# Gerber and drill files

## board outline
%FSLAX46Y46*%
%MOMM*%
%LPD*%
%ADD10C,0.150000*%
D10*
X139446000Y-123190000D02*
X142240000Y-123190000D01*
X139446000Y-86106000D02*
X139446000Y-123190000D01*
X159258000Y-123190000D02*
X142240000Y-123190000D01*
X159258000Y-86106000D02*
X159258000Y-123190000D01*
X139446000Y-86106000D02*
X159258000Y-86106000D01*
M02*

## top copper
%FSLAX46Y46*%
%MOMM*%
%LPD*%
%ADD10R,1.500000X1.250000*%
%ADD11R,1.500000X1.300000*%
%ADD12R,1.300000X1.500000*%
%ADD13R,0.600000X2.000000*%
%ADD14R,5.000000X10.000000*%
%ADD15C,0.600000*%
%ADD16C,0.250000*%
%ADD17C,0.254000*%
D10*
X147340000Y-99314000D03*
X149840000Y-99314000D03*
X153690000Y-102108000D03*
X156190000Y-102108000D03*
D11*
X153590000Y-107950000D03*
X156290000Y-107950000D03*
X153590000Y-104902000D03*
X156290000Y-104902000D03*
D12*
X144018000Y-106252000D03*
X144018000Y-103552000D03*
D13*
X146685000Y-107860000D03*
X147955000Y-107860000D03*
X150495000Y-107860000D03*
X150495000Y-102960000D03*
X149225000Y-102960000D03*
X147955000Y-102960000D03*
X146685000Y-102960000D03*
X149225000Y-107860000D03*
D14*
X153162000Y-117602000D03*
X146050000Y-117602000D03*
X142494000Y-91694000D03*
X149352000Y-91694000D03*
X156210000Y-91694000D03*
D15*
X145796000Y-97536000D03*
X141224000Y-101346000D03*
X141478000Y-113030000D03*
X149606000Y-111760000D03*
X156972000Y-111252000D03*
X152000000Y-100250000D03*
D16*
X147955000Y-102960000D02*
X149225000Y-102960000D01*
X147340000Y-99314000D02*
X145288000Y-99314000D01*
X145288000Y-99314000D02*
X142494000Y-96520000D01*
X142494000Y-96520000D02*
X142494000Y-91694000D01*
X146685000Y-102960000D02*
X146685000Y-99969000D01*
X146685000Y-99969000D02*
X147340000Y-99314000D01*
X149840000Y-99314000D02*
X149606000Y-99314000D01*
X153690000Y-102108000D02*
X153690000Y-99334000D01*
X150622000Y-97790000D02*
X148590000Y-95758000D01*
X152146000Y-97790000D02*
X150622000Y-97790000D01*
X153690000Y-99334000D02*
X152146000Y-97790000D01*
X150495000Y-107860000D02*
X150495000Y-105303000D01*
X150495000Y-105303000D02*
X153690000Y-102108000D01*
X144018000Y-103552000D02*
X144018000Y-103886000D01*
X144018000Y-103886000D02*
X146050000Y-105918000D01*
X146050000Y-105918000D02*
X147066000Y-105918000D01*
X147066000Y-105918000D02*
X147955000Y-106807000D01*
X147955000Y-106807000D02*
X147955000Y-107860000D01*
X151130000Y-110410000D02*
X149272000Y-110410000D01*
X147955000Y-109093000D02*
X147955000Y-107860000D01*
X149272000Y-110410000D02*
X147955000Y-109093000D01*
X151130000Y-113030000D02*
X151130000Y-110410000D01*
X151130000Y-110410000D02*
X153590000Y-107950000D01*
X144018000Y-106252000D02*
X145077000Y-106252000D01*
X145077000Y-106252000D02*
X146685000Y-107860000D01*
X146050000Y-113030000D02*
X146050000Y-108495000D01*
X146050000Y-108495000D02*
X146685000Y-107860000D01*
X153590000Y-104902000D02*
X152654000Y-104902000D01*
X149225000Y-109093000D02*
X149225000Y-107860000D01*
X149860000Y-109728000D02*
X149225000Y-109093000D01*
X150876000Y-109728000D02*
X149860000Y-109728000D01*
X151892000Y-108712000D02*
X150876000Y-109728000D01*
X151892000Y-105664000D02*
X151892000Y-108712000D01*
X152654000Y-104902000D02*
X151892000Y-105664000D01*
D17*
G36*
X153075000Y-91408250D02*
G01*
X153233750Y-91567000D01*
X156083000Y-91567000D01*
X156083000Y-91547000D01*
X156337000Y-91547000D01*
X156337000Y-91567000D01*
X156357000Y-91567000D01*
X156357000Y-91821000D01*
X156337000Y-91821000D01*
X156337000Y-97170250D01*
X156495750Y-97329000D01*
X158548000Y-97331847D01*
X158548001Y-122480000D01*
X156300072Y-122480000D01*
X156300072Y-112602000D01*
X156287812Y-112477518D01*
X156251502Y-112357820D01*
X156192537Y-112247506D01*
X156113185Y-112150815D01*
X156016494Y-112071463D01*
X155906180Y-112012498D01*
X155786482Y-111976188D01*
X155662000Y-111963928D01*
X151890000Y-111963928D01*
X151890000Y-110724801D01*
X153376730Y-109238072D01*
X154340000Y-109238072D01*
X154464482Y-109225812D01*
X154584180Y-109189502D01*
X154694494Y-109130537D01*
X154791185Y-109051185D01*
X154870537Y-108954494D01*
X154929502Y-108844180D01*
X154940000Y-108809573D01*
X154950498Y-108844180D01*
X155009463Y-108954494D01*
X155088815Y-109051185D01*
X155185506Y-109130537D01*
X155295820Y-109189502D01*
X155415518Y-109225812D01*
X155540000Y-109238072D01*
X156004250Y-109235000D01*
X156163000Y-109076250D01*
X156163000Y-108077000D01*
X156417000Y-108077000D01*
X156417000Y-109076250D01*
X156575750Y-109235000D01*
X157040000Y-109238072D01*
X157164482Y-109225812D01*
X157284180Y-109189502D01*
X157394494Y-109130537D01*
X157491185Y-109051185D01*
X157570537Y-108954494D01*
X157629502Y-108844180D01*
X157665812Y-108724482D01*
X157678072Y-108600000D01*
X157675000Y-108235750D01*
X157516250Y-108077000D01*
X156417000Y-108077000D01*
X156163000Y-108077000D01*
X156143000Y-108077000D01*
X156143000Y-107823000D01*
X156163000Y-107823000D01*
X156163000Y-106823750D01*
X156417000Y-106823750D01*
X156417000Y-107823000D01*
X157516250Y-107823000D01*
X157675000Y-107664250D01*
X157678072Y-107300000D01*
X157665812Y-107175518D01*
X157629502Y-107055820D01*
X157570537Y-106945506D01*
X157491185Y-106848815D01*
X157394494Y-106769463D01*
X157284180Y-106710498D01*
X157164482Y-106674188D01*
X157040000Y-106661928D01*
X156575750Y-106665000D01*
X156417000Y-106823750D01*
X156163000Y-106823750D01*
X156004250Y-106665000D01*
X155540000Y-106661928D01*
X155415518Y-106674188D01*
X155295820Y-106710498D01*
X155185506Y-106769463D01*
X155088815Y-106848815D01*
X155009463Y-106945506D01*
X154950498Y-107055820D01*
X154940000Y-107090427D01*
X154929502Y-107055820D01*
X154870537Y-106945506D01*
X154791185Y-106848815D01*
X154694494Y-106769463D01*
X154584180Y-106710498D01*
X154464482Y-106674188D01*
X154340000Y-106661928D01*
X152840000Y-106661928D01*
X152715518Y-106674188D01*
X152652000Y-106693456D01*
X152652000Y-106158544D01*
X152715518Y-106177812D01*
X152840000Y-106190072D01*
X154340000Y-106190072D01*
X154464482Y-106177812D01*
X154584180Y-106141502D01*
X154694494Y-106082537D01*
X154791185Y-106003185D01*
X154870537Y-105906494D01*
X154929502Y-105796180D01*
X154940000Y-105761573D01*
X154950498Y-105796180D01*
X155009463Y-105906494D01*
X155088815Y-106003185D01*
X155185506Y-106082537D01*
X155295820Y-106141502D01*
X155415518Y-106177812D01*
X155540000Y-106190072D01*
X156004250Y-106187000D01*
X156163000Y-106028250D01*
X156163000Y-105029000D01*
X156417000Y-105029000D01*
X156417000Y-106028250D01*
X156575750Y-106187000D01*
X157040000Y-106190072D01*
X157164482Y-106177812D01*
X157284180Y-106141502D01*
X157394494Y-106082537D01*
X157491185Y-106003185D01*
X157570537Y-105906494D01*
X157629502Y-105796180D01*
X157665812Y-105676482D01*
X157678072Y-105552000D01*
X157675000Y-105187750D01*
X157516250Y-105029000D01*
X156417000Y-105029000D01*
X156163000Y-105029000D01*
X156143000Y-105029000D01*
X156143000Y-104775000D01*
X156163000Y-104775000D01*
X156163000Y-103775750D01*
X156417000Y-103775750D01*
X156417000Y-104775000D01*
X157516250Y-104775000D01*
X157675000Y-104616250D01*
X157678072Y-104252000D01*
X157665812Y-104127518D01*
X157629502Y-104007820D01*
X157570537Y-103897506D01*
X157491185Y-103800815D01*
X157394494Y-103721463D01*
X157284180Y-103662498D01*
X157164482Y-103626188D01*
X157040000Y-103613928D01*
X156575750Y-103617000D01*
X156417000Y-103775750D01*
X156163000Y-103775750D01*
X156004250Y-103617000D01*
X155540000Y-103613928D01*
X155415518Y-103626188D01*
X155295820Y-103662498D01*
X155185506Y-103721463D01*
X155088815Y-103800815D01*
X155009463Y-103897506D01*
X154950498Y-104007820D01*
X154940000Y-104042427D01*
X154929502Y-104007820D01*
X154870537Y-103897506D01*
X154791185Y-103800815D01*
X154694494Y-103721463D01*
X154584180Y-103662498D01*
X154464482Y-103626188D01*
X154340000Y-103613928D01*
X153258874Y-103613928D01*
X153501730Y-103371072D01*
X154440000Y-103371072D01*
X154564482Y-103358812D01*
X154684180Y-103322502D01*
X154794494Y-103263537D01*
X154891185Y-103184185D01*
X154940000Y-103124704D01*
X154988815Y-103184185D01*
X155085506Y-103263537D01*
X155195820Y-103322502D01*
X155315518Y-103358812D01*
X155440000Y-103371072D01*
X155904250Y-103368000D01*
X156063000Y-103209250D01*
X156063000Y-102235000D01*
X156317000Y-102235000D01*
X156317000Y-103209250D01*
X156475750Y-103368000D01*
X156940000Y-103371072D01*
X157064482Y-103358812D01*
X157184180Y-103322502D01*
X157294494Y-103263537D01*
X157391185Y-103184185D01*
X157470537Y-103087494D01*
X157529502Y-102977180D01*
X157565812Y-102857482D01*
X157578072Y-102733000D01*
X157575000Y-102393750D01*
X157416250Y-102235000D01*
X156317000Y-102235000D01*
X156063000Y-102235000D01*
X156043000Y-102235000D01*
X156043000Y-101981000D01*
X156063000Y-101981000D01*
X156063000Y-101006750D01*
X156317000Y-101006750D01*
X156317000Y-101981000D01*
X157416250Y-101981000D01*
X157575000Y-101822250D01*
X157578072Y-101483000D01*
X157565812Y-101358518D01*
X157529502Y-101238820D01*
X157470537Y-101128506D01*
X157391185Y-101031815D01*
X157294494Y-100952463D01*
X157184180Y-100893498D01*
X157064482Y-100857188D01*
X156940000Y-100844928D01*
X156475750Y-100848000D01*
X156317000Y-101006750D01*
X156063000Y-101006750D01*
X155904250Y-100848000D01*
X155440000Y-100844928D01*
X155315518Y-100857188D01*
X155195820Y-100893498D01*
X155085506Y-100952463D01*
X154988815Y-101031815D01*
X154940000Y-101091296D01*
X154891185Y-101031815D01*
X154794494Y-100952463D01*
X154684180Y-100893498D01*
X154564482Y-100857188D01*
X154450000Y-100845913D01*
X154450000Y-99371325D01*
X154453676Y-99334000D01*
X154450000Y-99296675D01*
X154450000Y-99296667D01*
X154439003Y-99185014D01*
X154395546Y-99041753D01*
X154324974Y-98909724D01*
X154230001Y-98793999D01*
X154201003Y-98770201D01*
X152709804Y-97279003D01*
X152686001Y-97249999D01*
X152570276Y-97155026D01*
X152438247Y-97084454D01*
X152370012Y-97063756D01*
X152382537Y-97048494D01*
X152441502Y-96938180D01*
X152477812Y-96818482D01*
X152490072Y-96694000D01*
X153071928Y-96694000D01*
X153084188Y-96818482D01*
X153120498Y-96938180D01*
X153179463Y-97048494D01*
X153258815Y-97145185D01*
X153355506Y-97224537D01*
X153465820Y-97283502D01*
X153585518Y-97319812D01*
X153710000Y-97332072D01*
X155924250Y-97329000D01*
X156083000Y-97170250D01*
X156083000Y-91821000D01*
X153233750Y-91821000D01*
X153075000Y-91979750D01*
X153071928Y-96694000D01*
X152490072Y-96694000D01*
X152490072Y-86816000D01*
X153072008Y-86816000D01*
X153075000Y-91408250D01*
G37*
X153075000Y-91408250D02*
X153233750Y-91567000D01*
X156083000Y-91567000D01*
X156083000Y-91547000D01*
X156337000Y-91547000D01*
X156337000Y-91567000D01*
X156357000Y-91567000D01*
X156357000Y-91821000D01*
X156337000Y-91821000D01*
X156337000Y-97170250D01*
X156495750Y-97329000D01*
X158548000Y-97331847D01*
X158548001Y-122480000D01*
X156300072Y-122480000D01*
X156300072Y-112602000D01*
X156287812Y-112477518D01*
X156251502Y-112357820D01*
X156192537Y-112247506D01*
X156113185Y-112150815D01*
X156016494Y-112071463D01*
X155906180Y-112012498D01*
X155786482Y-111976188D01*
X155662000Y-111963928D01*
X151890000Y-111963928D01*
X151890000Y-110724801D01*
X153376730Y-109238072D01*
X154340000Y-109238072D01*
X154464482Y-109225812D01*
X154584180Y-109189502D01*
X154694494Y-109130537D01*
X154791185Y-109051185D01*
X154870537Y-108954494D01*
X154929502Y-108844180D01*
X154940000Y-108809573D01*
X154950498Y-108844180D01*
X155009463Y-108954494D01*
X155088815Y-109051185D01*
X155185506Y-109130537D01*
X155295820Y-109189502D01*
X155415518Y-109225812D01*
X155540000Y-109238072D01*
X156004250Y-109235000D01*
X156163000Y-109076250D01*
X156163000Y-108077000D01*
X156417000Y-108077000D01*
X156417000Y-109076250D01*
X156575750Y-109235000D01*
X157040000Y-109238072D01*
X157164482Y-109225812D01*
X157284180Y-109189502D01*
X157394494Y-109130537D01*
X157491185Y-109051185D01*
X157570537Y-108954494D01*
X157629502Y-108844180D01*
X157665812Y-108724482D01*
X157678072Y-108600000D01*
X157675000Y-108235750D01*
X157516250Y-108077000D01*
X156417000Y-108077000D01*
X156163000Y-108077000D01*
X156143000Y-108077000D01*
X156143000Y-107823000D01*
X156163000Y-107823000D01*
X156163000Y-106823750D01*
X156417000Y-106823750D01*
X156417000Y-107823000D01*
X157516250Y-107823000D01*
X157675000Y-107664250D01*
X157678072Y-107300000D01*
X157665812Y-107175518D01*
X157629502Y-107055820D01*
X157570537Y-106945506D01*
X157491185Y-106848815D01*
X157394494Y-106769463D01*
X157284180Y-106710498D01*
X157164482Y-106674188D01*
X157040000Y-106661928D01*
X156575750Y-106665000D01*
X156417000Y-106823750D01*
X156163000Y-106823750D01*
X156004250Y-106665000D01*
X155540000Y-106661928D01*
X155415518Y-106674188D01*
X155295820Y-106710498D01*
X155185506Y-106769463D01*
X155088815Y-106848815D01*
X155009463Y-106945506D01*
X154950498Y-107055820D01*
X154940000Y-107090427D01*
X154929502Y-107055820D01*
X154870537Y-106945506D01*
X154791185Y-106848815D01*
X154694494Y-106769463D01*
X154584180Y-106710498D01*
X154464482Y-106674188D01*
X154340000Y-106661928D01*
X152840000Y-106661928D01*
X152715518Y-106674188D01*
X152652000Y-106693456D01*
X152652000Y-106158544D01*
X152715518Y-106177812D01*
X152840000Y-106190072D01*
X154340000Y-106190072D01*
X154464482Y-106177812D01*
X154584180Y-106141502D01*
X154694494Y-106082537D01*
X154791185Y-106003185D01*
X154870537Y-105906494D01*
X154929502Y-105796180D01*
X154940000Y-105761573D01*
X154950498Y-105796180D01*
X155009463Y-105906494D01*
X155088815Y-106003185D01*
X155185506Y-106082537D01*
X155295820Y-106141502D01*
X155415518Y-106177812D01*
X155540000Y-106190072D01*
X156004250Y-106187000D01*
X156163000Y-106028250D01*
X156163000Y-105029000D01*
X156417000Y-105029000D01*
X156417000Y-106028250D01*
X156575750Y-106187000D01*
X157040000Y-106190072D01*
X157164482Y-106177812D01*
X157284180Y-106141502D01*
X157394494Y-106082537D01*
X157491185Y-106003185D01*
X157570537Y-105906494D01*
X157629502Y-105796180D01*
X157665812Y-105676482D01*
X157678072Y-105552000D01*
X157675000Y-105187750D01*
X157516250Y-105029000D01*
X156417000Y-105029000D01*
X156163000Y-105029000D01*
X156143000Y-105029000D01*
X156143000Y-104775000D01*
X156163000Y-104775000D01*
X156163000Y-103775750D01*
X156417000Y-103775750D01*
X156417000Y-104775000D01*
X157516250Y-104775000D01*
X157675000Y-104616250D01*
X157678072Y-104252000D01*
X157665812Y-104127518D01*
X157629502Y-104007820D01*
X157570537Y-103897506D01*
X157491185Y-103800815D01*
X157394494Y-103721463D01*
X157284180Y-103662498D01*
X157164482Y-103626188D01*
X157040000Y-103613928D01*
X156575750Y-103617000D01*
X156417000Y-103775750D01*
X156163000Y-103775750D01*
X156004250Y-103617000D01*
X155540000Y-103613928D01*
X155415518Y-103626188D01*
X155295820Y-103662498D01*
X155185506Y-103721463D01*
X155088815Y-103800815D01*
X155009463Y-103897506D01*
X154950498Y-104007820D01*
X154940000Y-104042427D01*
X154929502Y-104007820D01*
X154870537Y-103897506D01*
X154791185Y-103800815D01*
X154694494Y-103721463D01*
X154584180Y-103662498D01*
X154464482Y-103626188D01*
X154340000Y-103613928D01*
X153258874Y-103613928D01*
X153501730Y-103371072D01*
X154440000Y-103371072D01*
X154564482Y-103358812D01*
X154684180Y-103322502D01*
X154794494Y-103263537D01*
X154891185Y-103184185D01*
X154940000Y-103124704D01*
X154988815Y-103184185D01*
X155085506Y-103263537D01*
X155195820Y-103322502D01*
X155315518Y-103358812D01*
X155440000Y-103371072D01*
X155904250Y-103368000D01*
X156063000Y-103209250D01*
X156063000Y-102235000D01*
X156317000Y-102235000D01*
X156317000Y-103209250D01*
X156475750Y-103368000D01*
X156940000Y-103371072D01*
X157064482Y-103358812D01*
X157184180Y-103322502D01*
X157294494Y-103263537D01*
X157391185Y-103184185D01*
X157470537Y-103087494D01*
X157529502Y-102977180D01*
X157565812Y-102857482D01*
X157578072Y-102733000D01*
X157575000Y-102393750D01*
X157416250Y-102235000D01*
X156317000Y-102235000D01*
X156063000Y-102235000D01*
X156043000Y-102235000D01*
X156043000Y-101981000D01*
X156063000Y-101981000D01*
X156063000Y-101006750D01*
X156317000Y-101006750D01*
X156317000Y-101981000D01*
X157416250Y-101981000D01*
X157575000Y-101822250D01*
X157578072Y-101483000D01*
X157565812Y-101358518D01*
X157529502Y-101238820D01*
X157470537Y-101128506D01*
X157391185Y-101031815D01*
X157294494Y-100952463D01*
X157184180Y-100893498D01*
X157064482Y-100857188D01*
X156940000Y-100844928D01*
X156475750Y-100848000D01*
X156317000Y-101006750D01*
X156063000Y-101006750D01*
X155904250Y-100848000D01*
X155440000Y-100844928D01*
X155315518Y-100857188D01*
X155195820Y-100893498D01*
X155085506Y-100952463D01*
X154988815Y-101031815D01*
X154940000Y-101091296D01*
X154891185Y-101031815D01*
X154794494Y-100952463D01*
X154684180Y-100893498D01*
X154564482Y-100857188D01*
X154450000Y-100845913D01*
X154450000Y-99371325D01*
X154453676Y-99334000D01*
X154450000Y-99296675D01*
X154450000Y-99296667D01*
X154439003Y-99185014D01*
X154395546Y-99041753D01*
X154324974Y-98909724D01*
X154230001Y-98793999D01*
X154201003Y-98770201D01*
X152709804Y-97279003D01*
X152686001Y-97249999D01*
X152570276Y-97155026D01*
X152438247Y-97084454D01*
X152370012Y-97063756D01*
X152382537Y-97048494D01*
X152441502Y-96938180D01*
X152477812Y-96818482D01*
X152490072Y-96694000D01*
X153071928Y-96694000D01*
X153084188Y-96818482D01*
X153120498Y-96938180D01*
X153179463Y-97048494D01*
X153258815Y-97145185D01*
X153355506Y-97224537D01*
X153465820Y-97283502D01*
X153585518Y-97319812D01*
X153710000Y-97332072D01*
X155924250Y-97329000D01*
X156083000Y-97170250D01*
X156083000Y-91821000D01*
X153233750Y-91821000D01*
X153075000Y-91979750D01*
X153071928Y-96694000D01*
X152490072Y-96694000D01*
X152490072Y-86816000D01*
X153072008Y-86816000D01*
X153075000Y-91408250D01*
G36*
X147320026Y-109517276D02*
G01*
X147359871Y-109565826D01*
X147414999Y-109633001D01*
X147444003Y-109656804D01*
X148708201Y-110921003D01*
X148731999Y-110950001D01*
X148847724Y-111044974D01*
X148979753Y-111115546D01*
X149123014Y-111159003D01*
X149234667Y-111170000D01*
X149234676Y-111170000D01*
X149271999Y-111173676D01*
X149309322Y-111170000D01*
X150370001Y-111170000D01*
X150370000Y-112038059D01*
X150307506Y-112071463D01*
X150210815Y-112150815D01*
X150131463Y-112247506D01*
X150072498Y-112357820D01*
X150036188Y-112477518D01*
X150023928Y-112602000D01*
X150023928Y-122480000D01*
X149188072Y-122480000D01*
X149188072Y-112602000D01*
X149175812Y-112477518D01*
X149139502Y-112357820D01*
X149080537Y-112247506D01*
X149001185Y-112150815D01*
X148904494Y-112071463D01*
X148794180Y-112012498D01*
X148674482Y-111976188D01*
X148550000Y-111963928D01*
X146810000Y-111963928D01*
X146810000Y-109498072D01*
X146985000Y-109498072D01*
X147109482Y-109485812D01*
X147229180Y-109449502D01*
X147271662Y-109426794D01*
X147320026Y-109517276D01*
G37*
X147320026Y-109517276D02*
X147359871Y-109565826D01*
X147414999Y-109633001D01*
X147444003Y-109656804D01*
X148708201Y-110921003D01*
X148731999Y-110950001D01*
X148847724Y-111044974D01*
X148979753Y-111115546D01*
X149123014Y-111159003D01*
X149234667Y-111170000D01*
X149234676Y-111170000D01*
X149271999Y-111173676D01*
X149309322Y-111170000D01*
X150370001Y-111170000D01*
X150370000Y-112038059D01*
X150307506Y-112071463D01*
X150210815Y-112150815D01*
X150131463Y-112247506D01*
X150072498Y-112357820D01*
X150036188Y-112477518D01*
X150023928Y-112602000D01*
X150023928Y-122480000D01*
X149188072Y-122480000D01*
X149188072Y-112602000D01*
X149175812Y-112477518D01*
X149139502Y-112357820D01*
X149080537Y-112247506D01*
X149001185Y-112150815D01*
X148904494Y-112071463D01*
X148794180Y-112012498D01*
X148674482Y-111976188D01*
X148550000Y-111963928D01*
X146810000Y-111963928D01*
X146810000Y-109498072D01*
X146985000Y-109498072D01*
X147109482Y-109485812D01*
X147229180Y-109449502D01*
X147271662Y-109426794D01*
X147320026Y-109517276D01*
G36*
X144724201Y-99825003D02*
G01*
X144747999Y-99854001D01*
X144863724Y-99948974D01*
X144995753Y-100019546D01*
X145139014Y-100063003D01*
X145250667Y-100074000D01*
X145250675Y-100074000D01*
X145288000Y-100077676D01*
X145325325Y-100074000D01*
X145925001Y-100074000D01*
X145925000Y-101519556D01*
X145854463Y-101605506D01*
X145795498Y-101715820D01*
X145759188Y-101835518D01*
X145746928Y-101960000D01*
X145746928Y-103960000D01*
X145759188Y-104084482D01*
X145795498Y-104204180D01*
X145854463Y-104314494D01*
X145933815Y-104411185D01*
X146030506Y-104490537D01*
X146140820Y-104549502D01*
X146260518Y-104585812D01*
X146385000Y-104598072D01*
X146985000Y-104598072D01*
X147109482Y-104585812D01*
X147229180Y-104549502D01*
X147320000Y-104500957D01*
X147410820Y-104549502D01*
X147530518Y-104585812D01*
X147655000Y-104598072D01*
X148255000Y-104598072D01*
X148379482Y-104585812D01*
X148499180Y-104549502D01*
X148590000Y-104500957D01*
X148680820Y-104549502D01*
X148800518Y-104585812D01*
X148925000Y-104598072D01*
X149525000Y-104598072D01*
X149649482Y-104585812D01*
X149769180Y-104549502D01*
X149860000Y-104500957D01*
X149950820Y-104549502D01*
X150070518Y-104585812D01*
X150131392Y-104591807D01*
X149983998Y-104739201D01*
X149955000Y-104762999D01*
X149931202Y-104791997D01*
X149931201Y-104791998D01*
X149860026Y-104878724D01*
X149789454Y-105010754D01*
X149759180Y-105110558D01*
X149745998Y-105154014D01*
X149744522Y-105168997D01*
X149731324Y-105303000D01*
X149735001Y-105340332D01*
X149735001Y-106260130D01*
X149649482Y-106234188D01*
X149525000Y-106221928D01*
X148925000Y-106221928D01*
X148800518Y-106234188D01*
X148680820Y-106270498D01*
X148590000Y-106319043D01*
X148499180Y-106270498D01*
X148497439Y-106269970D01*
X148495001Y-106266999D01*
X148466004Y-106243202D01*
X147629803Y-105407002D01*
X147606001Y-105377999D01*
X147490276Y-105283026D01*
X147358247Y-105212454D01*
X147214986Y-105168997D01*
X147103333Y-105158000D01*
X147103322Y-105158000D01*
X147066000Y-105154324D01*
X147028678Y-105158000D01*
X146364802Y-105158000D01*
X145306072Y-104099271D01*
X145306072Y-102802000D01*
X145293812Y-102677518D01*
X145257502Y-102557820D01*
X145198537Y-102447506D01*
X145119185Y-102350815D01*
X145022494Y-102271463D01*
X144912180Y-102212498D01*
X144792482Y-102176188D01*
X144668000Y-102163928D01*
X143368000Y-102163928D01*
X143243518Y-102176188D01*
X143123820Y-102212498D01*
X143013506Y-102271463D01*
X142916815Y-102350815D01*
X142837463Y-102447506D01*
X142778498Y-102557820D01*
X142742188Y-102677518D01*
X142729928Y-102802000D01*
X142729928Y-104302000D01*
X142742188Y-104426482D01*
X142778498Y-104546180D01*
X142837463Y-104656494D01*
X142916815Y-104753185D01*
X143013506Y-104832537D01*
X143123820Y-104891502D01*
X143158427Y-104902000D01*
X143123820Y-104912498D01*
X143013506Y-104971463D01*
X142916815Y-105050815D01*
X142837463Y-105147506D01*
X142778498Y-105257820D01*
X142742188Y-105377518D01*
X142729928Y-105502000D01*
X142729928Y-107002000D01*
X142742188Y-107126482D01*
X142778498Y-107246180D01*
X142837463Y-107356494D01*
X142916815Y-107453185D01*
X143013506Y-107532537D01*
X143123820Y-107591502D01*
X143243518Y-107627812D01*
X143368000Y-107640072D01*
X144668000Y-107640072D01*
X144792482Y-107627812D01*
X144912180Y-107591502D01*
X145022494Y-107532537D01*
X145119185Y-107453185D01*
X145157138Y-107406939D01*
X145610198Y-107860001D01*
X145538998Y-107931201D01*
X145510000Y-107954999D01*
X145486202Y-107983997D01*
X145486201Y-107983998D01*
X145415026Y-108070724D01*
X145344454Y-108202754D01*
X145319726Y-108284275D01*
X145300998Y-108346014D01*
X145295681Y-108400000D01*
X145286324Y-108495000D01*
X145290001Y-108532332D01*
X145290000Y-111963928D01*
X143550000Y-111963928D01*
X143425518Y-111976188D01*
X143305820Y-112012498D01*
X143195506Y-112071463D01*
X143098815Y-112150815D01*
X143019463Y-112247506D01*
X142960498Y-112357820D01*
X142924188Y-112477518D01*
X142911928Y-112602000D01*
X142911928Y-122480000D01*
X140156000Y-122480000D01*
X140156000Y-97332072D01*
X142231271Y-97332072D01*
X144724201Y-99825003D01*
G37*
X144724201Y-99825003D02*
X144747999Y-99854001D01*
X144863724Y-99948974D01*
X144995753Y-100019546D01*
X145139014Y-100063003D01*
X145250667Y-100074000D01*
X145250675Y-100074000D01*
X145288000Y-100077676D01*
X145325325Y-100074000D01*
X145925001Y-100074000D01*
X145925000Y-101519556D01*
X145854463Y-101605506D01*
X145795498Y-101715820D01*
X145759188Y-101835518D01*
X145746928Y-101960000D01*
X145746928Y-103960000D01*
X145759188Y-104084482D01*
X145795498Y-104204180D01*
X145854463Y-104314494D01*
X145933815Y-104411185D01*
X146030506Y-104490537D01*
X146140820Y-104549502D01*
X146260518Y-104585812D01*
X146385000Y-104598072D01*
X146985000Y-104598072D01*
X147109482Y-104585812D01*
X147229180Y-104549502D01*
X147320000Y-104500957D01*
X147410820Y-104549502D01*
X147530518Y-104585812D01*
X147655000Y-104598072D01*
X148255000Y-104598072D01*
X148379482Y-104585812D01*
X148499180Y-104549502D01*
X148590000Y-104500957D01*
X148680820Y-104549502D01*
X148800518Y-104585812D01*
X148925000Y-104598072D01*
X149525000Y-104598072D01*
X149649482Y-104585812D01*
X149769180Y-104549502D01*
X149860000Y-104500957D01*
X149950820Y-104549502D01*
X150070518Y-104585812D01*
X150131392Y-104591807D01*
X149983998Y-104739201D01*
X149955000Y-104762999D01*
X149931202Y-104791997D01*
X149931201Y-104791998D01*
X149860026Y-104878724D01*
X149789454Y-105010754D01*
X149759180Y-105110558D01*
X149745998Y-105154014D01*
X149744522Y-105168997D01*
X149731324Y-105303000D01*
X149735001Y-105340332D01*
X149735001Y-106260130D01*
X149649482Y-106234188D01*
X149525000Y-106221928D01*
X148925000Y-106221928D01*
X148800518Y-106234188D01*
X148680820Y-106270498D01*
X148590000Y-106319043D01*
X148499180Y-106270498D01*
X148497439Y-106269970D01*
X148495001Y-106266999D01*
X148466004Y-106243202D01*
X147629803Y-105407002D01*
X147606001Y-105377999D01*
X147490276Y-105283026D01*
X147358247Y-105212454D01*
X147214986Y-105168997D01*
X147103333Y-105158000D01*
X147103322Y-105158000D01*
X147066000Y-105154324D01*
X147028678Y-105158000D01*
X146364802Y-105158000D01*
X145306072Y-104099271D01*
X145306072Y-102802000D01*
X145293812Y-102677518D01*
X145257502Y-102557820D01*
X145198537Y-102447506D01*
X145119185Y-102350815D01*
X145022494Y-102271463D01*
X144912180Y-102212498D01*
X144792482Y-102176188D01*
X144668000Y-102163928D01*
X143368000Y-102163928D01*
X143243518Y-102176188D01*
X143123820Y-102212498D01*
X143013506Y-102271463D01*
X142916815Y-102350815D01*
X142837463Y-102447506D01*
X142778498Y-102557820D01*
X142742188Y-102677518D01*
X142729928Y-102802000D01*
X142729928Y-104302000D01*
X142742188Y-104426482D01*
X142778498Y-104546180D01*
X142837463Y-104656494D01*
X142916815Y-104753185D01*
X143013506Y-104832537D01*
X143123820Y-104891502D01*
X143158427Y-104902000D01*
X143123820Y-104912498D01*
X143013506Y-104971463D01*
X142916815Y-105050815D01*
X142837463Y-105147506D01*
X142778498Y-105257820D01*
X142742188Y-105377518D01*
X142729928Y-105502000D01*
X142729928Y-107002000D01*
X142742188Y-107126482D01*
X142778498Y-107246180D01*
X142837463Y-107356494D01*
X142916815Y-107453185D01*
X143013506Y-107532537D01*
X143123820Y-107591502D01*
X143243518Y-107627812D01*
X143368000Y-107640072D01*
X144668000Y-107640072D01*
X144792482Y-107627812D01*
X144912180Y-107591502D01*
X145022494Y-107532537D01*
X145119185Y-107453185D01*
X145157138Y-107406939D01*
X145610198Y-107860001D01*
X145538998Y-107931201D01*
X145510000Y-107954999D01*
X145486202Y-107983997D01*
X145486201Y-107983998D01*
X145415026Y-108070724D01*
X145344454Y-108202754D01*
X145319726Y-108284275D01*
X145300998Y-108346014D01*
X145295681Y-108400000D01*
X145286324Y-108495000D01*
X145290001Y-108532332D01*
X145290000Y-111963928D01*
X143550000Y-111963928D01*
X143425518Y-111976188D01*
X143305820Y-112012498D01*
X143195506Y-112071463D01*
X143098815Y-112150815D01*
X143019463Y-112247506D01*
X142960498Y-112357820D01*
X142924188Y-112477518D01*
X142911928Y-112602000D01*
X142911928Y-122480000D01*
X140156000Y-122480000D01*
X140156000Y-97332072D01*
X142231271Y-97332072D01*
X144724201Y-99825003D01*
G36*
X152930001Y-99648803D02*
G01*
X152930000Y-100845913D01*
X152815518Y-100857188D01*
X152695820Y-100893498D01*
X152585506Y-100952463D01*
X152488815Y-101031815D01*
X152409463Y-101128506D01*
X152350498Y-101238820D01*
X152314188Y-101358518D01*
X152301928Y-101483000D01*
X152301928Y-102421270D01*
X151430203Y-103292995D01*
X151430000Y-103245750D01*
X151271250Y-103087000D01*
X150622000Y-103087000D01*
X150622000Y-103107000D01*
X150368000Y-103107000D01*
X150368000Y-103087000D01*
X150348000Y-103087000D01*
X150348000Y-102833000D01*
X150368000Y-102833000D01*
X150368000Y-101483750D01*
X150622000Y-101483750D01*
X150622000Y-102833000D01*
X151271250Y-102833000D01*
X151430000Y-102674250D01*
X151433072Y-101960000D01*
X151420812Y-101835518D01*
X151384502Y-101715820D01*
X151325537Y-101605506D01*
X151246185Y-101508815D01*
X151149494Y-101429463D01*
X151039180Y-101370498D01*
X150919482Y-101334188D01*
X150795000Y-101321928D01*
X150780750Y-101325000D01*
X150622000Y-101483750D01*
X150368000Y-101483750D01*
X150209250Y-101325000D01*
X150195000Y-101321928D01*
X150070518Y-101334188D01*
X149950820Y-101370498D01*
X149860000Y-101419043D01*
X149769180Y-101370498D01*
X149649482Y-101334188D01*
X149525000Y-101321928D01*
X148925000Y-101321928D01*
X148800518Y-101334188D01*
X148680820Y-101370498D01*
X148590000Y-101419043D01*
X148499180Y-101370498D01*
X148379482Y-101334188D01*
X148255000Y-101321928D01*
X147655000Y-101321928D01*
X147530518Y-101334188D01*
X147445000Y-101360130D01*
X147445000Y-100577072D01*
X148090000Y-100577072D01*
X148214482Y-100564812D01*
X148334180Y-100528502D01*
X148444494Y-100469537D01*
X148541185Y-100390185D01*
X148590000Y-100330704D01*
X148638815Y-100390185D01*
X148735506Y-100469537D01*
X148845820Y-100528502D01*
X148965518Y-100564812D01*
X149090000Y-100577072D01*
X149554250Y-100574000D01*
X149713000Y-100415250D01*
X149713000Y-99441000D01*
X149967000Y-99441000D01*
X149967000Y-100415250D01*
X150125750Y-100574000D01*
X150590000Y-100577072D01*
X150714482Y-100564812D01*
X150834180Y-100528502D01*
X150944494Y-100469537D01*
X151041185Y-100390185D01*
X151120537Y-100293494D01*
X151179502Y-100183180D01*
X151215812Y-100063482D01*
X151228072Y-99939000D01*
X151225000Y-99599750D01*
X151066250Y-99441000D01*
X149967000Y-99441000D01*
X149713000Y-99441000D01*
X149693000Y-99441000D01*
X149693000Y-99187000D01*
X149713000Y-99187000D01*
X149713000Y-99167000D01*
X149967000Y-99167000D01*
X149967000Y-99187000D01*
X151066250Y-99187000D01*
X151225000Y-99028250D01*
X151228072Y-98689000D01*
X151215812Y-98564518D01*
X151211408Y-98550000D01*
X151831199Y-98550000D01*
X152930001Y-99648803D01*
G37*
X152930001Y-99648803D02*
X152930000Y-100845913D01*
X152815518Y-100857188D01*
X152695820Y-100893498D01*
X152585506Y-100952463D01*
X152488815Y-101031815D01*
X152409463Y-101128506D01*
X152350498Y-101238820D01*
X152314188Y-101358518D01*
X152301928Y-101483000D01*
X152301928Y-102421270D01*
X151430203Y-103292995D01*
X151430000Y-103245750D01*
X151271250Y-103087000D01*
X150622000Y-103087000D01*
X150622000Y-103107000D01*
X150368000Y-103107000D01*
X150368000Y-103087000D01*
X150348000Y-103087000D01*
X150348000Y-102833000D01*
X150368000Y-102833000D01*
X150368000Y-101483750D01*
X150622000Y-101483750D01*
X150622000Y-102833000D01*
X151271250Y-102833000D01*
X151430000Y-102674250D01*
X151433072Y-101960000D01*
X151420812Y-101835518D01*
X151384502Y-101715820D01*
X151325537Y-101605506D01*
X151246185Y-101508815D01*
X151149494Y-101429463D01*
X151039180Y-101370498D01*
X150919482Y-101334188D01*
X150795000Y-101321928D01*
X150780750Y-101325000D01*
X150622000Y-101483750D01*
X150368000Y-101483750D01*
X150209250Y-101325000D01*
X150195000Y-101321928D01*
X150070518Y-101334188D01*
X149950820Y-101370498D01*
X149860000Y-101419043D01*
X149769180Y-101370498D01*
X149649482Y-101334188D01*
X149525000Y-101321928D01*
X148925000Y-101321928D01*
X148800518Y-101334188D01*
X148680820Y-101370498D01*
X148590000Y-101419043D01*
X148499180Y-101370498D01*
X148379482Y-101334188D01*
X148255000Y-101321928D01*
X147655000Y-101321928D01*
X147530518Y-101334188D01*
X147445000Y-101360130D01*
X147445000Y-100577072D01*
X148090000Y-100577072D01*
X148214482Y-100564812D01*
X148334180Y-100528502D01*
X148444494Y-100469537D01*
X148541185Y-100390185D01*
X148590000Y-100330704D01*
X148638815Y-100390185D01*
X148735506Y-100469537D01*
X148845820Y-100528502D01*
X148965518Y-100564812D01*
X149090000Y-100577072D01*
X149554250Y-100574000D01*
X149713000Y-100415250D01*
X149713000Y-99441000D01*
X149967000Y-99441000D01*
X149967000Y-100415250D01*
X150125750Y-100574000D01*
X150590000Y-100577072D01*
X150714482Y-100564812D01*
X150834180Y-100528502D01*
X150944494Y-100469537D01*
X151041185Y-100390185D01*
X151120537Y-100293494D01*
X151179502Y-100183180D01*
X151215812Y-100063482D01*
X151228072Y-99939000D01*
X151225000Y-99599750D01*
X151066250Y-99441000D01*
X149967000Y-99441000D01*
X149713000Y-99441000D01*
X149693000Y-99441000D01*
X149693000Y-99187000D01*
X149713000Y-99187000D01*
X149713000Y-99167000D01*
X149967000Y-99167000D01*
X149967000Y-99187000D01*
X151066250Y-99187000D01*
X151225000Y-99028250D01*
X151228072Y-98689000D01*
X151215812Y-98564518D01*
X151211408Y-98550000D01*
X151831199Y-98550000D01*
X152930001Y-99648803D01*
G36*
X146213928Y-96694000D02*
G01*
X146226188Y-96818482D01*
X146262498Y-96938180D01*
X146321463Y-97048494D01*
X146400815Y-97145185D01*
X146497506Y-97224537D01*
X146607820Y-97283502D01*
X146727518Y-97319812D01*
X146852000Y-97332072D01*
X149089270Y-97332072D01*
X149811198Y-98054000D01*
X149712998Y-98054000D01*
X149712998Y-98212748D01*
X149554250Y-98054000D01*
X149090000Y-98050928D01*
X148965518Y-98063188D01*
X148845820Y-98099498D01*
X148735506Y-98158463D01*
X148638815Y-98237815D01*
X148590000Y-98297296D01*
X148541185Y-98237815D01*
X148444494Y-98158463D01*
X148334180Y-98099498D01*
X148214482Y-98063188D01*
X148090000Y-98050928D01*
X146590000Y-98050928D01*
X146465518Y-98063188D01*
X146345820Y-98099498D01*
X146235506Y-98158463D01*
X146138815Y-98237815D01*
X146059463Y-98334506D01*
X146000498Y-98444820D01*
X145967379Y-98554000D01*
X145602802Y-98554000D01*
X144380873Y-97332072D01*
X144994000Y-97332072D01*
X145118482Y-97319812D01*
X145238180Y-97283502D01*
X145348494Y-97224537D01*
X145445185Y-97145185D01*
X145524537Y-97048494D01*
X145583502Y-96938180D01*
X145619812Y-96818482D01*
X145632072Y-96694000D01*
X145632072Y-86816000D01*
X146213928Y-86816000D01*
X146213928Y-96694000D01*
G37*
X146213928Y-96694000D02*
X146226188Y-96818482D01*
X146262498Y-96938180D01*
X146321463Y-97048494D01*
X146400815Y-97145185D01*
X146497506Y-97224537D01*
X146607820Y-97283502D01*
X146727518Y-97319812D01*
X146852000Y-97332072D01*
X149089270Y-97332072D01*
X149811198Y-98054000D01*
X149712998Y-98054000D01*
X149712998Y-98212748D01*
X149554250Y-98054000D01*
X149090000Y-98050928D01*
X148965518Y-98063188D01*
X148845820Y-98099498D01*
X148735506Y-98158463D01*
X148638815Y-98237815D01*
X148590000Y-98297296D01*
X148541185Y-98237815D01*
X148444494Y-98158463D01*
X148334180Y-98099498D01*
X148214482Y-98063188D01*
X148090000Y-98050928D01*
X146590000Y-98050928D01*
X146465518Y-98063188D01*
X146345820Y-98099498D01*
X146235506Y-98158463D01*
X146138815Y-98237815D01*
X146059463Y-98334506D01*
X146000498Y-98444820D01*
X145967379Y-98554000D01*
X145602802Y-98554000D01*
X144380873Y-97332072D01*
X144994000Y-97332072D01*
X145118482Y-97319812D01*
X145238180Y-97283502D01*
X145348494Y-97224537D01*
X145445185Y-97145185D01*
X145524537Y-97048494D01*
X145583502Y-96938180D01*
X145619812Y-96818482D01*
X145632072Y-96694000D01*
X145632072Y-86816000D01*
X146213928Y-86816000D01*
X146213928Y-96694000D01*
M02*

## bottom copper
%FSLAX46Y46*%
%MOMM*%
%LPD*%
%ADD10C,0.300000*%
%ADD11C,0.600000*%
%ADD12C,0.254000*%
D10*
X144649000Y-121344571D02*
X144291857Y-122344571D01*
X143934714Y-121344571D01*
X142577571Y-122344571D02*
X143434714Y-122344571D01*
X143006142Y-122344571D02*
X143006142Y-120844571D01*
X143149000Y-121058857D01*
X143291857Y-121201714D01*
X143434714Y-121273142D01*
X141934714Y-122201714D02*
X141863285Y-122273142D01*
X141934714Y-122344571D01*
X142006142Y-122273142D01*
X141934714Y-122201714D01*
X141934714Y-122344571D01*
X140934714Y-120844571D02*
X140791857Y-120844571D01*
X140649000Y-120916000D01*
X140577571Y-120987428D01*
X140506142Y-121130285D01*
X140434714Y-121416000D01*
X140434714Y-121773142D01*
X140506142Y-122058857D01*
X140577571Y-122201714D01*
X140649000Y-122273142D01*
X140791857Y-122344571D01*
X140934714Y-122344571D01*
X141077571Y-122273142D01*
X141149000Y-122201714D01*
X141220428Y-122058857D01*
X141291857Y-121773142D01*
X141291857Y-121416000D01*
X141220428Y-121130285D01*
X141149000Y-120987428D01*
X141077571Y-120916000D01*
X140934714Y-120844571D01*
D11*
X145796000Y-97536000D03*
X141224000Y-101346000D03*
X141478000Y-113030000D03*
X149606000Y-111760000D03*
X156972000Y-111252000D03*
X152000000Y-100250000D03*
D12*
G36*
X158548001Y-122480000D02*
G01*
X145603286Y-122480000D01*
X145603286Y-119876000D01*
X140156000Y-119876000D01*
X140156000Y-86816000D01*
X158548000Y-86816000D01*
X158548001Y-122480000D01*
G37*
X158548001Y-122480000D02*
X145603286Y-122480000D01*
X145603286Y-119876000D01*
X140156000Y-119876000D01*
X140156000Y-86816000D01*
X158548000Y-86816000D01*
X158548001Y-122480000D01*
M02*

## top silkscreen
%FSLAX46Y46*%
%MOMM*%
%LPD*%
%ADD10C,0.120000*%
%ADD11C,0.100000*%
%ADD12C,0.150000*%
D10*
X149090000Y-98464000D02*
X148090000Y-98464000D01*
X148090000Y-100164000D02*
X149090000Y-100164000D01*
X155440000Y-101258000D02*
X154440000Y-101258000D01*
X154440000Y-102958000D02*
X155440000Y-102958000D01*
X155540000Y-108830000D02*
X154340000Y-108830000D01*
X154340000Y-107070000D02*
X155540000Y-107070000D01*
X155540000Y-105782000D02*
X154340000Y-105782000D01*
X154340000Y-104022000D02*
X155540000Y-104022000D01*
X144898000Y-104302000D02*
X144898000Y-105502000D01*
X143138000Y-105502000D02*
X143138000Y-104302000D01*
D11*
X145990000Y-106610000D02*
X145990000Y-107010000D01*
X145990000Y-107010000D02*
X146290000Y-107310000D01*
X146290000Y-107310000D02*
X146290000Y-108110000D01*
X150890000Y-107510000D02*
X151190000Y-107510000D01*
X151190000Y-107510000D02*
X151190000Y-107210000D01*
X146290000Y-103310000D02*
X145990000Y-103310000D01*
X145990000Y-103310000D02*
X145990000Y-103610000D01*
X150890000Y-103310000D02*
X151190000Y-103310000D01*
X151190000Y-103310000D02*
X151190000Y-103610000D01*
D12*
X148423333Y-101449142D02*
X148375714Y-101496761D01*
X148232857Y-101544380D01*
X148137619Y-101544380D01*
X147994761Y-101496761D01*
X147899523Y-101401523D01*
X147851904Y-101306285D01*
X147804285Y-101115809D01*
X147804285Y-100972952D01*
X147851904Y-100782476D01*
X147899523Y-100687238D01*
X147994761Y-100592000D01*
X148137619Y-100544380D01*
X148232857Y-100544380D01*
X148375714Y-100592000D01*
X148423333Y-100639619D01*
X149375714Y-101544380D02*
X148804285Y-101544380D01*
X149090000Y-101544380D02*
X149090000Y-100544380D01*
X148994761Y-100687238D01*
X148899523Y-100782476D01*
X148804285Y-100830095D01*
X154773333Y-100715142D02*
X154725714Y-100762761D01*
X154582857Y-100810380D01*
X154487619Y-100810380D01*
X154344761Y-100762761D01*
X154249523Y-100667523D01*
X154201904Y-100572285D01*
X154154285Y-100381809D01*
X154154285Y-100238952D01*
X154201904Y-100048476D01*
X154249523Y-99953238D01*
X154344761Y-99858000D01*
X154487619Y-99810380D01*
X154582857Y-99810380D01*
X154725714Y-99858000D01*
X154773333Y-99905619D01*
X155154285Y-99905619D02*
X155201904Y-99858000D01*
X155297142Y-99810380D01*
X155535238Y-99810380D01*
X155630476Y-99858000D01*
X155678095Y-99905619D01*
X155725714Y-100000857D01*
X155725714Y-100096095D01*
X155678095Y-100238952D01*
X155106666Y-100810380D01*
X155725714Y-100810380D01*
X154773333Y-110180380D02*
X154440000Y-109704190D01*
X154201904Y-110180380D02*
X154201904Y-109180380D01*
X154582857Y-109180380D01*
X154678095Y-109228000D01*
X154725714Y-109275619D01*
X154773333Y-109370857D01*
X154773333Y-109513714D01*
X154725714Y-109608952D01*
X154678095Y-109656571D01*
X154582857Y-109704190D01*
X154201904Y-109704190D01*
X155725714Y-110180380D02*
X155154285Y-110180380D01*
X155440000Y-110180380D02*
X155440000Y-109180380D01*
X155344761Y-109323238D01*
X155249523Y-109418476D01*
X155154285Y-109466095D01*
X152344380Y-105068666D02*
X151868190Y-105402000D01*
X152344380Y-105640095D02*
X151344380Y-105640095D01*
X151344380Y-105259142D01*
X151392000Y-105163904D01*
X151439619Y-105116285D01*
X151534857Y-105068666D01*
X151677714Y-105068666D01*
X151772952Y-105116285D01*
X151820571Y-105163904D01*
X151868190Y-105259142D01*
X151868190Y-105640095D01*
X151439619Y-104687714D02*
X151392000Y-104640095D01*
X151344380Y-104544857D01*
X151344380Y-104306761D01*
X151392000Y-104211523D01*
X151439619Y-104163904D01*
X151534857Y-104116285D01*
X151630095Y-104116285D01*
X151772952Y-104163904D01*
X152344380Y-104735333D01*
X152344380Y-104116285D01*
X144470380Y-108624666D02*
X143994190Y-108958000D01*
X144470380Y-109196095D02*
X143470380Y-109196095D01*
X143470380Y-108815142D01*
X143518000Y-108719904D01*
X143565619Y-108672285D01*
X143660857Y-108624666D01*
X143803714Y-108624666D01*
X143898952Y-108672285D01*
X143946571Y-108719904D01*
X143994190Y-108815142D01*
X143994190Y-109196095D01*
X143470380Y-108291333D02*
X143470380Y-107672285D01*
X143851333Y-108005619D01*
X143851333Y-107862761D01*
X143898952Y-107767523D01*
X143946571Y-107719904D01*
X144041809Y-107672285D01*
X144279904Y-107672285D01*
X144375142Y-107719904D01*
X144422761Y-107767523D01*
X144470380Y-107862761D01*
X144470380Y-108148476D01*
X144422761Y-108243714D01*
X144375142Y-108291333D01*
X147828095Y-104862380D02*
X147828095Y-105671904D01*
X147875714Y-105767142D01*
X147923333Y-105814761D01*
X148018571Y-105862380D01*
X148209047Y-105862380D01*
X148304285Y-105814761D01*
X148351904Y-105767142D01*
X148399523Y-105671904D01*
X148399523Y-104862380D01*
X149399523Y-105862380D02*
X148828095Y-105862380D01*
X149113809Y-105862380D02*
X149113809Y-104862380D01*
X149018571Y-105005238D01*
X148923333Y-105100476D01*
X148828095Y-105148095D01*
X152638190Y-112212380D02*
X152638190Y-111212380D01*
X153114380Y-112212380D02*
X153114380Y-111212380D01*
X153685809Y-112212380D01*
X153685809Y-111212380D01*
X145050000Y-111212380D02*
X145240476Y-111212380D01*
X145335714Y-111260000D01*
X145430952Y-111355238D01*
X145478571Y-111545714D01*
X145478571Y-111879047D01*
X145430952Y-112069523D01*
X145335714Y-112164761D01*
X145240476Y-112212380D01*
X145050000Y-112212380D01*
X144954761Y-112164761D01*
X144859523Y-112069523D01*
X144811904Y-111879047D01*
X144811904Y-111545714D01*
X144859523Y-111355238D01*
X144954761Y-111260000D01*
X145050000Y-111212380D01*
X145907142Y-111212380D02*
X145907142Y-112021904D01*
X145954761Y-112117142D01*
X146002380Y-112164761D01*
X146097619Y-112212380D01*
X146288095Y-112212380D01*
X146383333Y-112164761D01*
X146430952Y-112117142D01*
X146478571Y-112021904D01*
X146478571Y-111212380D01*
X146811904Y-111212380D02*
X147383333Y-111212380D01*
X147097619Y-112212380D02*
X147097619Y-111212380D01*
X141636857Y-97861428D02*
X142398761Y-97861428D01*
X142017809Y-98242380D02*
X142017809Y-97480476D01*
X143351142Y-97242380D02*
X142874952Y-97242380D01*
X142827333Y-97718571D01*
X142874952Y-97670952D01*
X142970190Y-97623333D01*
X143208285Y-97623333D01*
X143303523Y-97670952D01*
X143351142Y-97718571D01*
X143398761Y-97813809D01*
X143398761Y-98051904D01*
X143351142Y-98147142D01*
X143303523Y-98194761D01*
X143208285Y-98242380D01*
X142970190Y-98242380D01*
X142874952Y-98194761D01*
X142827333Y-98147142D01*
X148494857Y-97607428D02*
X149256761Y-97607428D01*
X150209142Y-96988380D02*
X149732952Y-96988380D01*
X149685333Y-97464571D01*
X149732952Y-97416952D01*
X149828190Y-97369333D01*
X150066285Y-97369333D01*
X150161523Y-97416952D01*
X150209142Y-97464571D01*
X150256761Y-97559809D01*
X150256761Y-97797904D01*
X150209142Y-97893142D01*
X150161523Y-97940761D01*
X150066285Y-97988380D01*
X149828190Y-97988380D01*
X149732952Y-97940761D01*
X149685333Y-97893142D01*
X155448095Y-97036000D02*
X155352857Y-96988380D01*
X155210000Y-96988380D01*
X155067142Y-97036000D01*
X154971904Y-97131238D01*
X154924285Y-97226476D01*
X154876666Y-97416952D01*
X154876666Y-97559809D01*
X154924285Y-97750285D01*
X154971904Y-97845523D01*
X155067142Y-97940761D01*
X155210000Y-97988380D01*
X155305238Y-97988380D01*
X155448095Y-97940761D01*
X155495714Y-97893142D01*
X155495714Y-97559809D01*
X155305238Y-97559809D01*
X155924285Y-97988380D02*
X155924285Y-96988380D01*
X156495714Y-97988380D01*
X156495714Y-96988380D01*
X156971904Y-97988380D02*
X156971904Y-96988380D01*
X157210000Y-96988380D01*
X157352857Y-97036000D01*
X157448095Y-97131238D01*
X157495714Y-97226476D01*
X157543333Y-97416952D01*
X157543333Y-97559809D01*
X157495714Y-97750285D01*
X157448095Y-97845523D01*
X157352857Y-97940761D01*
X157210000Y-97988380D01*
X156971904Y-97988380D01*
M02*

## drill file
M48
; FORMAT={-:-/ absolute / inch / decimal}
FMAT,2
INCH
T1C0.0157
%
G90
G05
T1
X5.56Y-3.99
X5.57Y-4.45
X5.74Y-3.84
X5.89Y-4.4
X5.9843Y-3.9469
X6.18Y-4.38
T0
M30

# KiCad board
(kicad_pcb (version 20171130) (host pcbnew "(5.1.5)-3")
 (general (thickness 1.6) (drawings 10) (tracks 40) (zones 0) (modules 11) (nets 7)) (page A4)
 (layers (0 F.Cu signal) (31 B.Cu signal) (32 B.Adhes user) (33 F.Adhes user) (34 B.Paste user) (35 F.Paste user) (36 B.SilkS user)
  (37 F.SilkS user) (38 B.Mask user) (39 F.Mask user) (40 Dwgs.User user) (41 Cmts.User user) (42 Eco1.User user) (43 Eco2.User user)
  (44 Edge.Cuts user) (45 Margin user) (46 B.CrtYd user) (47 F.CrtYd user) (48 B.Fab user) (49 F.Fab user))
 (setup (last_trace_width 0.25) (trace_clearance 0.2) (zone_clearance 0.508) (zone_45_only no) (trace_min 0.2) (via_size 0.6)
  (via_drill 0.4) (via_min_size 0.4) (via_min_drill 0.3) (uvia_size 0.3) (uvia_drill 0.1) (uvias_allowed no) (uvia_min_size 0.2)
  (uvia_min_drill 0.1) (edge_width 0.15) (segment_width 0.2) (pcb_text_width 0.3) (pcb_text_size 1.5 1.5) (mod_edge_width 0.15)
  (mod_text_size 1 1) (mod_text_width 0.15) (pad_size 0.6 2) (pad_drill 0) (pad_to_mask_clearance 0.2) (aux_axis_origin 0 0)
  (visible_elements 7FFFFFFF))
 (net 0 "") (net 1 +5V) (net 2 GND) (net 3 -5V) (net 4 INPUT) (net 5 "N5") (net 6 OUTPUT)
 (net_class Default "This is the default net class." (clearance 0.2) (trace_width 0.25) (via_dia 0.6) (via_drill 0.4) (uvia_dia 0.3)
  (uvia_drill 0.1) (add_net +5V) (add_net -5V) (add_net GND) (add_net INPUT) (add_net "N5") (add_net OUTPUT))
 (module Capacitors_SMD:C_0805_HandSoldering (layer F.Cu) (at 148.59 99.314)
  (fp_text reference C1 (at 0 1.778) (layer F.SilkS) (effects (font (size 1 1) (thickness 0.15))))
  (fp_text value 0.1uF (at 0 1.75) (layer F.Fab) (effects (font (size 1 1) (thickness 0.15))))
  (fp_line (start 0.5 -0.85) (end -0.5 -0.85) (layer F.SilkS) (width 0.12))
  (fp_line (start -0.5 0.85) (end 0.5 0.85) (layer F.SilkS) (width 0.12))
  (pad 1 smd rect (at -1.25 0) (size 1.5 1.25) (layers F.Cu F.Paste F.Mask) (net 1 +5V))
  (pad 2 smd rect (at 1.25 0) (size 1.5 1.25) (layers F.Cu F.Paste F.Mask) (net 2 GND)))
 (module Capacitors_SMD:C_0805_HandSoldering (layer F.Cu) (at 154.94 102.108)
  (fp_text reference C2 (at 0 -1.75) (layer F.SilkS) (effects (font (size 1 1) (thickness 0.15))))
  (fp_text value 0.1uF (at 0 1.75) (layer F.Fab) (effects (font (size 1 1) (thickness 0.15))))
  (fp_line (start 0.5 -0.85) (end -0.5 -0.85) (layer F.SilkS) (width 0.12))
  (fp_line (start -0.5 0.85) (end 0.5 0.85) (layer F.SilkS) (width 0.12))
  (pad 1 smd rect (at -1.25 0) (size 1.5 1.25) (layers F.Cu F.Paste F.Mask) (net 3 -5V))
  (pad 2 smd rect (at 1.25 0) (size 1.5 1.25) (layers F.Cu F.Paste F.Mask) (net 2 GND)))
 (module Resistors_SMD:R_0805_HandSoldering (layer F.Cu) (at 154.94 107.95)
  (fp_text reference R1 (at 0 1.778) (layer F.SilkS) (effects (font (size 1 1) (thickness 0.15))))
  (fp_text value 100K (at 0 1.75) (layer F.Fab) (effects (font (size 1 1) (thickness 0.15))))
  (fp_line (start 0.6 0.88) (end -0.6 0.88) (layer F.SilkS) (width 0.12))
  (fp_line (start -0.6 -0.88) (end 0.6 -0.88) (layer F.SilkS) (width 0.12))
  (pad 1 smd rect (at -1.35 0) (size 1.5 1.3) (layers F.Cu F.Paste F.Mask) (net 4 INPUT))
  (pad 2 smd rect (at 1.35 0) (size 1.5 1.3) (layers F.Cu F.Paste F.Mask) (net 2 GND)))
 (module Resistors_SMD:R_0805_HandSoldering (layer F.Cu) (at 154.94 104.902)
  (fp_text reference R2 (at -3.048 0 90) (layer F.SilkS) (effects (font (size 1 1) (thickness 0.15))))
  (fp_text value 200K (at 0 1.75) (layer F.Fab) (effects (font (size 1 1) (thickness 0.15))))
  (fp_line (start 0.6 0.88) (end -0.6 0.88) (layer F.SilkS) (width 0.12))
  (fp_line (start -0.6 -0.88) (end 0.6 -0.88) (layer F.SilkS) (width 0.12))
  (pad 1 smd rect (at -1.35 0) (size 1.5 1.3) (layers F.Cu F.Paste F.Mask) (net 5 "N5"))
  (pad 2 smd rect (at 1.35 0) (size 1.5 1.3) (layers F.Cu F.Paste F.Mask) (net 2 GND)))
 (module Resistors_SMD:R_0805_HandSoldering (layer F.Cu) (at 144.018 104.902 90)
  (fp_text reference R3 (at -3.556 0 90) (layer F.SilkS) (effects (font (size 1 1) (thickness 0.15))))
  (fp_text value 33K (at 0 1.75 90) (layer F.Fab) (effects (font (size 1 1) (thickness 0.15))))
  (fp_line (start 0.6 0.88) (end -0.6 0.88) (layer F.SilkS) (width 0.12))
  (fp_line (start -0.6 -0.88) (end 0.6 -0.88) (layer F.SilkS) (width 0.12))
  (pad 1 smd rect (at -1.35 0 90) (size 1.5 1.3) (layers F.Cu F.Paste F.Mask) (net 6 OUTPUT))
  (pad 2 smd rect (at 1.35 0 90) (size 1.5 1.3) (layers F.Cu F.Paste F.Mask) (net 4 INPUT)))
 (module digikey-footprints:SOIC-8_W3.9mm (layer F.Cu) (at 148.59 105.41)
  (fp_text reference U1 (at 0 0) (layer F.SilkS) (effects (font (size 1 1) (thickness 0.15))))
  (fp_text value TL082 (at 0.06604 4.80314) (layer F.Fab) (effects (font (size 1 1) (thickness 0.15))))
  (fp_line (start -2.6 1.2) (end -2.6 1.6) (layer F.SilkS) (width 0.1))
  (fp_line (start -2.6 1.6) (end -2.3 1.9) (layer F.SilkS) (width 0.1))
  (fp_line (start -2.3 1.9) (end -2.3 2.7) (layer F.SilkS) (width 0.1))
  (fp_line (start 2.3 2.1) (end 2.6 2.1) (layer F.SilkS) (width 0.1))
  (fp_line (start 2.6 2.1) (end 2.6 1.8) (layer F.SilkS) (width 0.1))
  (fp_line (start -2.3 -2.1) (end -2.6 -2.1) (layer F.SilkS) (width 0.1))
  (fp_line (start -2.6 -2.1) (end -2.6 -1.8) (layer F.SilkS) (width 0.1))
  (fp_line (start 2.3 -2.1) (end 2.6 -2.1) (layer F.SilkS) (width 0.1))
  (fp_line (start 2.6 -2.1) (end 2.6 -1.8) (layer F.SilkS) (width 0.1))
  (pad 1 smd rect (at -1.905 2.45) (size 0.6 2) (layers F.Cu F.Paste F.Mask) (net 6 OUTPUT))
  (pad 2 smd rect (at -0.635 2.45) (size 0.6 2) (layers F.Cu F.Paste F.Mask) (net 4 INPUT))
  (pad 4 smd rect (at 1.905 2.45) (size 0.6 2) (layers F.Cu F.Paste F.Mask) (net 3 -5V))
  (pad 5 smd rect (at 1.905 -2.45) (size 0.6 2) (layers F.Cu F.Paste F.Mask) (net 2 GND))
  (pad 6 smd rect (at 0.635 -2.45) (size 0.6 2) (layers F.Cu F.Paste F.Mask))
  (pad 7 smd rect (at -0.635 -2.45) (size 0.6 2) (layers F.Cu F.Paste F.Mask))
  (pad 8 smd rect (at -1.905 -2.45) (size 0.6 2) (layers F.Cu F.Paste F.Mask) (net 1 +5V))
  (pad 3 smd rect (at 0.635 2.45) (size 0.6 2) (layers F.Cu F.Paste F.Mask) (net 5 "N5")))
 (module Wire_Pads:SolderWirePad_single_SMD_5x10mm (layer F.Cu) (at 153.162 117.602)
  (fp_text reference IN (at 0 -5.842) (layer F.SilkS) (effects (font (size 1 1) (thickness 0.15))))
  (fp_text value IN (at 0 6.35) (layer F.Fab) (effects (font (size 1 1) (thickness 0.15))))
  (pad 1 smd rect (at 0 0) (size 5 10) (layers F.Cu F.Paste F.Mask) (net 4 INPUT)))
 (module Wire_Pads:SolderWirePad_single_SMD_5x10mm (layer F.Cu) (at 146.05 117.602)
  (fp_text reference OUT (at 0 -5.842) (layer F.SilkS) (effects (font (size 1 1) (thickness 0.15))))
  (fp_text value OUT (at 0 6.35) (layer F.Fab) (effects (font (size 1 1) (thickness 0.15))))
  (pad 1 smd rect (at 0 0) (size 5 10) (layers F.Cu F.Paste F.Mask) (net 6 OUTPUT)))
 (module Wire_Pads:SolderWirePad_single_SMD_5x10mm (layer F.Cu) (at 142.494 91.694)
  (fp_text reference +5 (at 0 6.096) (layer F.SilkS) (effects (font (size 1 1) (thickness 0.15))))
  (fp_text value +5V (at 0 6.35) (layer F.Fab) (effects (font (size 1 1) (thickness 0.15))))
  (pad 1 smd rect (at 0 0) (size 5 10) (layers F.Cu F.Paste F.Mask) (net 1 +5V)))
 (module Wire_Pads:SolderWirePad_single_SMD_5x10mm (layer F.Cu) (at 149.352 91.694)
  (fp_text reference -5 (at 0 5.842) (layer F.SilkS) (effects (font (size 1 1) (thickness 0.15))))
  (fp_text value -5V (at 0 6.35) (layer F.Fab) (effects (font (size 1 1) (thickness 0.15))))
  (pad 1 smd rect (at 0 0) (size 5 10) (layers F.Cu F.Paste F.Mask) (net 3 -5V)))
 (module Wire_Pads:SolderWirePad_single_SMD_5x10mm (layer F.Cu) (at 156.21 91.694)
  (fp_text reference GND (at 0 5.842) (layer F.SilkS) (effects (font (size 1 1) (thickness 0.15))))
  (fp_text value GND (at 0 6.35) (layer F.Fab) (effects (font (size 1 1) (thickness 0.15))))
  (pad 1 smd rect (at 0 0) (size 5 10) (layers F.Cu F.Paste F.Mask) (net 2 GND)))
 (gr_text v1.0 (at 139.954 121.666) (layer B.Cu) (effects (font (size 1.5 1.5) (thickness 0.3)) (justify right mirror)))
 (gr_line (start 139.446 123.19) (end 142.24 123.19) (angle 90) (layer Edge.Cuts) (width 0.15))
 (gr_line (start 139.446 86.106) (end 139.446 123.19) (angle 90) (layer Edge.Cuts) (width 0.15))
 (gr_line (start 159.258 123.19) (end 142.24 123.19) (angle 90) (layer Edge.Cuts) (width 0.15))
 (gr_line (start 159.258 86.106) (end 159.258 123.19) (angle 90) (layer Edge.Cuts) (width 0.15))
 (gr_line (start 139.446 86.106) (end 159.258 86.106) (angle 90) (layer Edge.Cuts) (width 0.15))
 (segment (start 147.955 102.96) (end 149.225 102.96) (width 0.25) (layer F.Cu) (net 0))
 (via (at 145.796 97.536) (size 0.6) (drill 0.4) (layers F.Cu B.Cu) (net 2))
 (via (at 141.224 101.346) (size 0.6) (drill 0.4) (layers F.Cu B.Cu) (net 2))
 (via (at 141.478 113.03) (size 0.6) (drill 0.4) (layers F.Cu B.Cu) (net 2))
 (via (at 149.606 111.76) (size 0.6) (drill 0.4) (layers F.Cu B.Cu) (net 2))
 (via (at 156.972 111.252) (size 0.6) (drill 0.4) (layers F.Cu B.Cu) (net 2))
 (segment (start 147.34 99.314) (end 145.288 99.314) (width 0.25) (layer F.Cu) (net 1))
 (segment (start 145.288 99.314) (end 142.494 96.52) (width 0.25) (layer F.Cu) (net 1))
 (segment (start 142.494 96.52) (end 142.494 91.694) (width 0.25) (layer F.Cu) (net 1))
 (segment (start 146.685 102.96) (end 146.685 99.969) (width 0.25) (layer F.Cu) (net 1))
 (segment (start 146.685 99.969) (end 147.34 99.314) (width 0.25) (layer F.Cu) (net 1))
 (segment (start 149.84 99.314) (end 149.606 99.314) (width 0.25) (layer F.Cu) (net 2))
 (via (at 152 100.25) (size 0.6) (drill 0.4) (layers F.Cu B.Cu) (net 2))
 (segment (start 153.69 102.108) (end 153.69 99.334) (width 0.25) (layer F.Cu) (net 3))
 (segment (start 150.622 97.79) (end 148.59 95.758) (width 0.25) (layer F.Cu) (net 3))
 (segment (start 152.146 97.79) (end 150.622 97.79) (width 0.25) (layer F.Cu) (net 3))
 (segment (start 153.69 99.334) (end 152.146 97.79) (width 0.25) (layer F.Cu) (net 3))
 (segment (start 150.495 107.86) (end 150.495 105.303) (width 0.25) (layer F.Cu) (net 3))
 (segment (start 150.495 105.303) (end 153.69 102.108) (width 0.25) (layer F.Cu) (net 3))
 (segment (start 144.018 103.552) (end 144.018 103.886) (width 0.25) (layer F.Cu) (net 4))
 (segment (start 144.018 103.886) (end 146.05 105.918) (width 0.25) (layer F.Cu) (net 4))
 (segment (start 146.05 105.918) (end 147.066 105.918) (width 0.25) (layer F.Cu) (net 4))
 (segment (start 147.066 105.918) (end 147.955 106.807) (width 0.25) (layer F.Cu) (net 4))
 (segment (start 147.955 106.807) (end 147.955 107.86) (width 0.25) (layer F.Cu) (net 4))
 (segment (start 151.13 110.41) (end 149.272 110.41) (width 0.25) (layer F.Cu) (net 4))
 (segment (start 147.955 109.093) (end 147.955 107.86) (width 0.25) (layer F.Cu) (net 4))
 (segment (start 149.272 110.41) (end 147.955 109.093) (width 0.25) (layer F.Cu) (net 4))
 (segment (start 151.13 113.03) (end 151.13 110.41) (width 0.25) (layer F.Cu) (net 4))
 (segment (start 151.13 110.41) (end 153.59 107.95) (width 0.25) (layer F.Cu) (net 4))
 (segment (start 144.018 106.252) (end 145.077 106.252) (width 0.25) (layer F.Cu) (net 6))
 (segment (start 145.077 106.252) (end 146.685 107.86) (width 0.25) (layer F.Cu) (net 6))
 (segment (start 146.05 113.03) (end 146.05 108.495) (width 0.25) (layer F.Cu) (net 6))
 (segment (start 146.05 108.495) (end 146.685 107.86) (width 0.25) (layer F.Cu) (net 6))
 (segment (start 153.59 104.902) (end 152.654 104.902) (width 0.25) (layer F.Cu) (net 5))
 (segment (start 149.225 109.093) (end 149.225 107.86) (width 0.25) (layer F.Cu) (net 5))
 (segment (start 149.86 109.728) (end 149.225 109.093) (width 0.25) (layer F.Cu) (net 5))
 (segment (start 150.876 109.728) (end 149.86 109.728) (width 0.25) (layer F.Cu) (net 5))
 (segment (start 151.892 108.712) (end 150.876 109.728) (width 0.25) (layer F.Cu) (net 5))
 (segment (start 151.892 105.664) (end 151.892 108.712) (width 0.25) (layer F.Cu) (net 5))
 (segment (start 152.654 104.902) (end 151.892 105.664) (width 0.25) (layer F.Cu) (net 5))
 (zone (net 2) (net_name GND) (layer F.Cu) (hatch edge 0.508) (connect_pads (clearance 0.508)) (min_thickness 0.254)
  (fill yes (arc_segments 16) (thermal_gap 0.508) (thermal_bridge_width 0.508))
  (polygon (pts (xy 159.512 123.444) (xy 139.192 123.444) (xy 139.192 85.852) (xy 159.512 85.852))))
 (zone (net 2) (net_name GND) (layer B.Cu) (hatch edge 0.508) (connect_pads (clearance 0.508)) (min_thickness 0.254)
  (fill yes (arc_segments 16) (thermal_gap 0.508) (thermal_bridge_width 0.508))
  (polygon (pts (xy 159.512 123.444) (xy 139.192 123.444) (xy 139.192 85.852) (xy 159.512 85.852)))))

